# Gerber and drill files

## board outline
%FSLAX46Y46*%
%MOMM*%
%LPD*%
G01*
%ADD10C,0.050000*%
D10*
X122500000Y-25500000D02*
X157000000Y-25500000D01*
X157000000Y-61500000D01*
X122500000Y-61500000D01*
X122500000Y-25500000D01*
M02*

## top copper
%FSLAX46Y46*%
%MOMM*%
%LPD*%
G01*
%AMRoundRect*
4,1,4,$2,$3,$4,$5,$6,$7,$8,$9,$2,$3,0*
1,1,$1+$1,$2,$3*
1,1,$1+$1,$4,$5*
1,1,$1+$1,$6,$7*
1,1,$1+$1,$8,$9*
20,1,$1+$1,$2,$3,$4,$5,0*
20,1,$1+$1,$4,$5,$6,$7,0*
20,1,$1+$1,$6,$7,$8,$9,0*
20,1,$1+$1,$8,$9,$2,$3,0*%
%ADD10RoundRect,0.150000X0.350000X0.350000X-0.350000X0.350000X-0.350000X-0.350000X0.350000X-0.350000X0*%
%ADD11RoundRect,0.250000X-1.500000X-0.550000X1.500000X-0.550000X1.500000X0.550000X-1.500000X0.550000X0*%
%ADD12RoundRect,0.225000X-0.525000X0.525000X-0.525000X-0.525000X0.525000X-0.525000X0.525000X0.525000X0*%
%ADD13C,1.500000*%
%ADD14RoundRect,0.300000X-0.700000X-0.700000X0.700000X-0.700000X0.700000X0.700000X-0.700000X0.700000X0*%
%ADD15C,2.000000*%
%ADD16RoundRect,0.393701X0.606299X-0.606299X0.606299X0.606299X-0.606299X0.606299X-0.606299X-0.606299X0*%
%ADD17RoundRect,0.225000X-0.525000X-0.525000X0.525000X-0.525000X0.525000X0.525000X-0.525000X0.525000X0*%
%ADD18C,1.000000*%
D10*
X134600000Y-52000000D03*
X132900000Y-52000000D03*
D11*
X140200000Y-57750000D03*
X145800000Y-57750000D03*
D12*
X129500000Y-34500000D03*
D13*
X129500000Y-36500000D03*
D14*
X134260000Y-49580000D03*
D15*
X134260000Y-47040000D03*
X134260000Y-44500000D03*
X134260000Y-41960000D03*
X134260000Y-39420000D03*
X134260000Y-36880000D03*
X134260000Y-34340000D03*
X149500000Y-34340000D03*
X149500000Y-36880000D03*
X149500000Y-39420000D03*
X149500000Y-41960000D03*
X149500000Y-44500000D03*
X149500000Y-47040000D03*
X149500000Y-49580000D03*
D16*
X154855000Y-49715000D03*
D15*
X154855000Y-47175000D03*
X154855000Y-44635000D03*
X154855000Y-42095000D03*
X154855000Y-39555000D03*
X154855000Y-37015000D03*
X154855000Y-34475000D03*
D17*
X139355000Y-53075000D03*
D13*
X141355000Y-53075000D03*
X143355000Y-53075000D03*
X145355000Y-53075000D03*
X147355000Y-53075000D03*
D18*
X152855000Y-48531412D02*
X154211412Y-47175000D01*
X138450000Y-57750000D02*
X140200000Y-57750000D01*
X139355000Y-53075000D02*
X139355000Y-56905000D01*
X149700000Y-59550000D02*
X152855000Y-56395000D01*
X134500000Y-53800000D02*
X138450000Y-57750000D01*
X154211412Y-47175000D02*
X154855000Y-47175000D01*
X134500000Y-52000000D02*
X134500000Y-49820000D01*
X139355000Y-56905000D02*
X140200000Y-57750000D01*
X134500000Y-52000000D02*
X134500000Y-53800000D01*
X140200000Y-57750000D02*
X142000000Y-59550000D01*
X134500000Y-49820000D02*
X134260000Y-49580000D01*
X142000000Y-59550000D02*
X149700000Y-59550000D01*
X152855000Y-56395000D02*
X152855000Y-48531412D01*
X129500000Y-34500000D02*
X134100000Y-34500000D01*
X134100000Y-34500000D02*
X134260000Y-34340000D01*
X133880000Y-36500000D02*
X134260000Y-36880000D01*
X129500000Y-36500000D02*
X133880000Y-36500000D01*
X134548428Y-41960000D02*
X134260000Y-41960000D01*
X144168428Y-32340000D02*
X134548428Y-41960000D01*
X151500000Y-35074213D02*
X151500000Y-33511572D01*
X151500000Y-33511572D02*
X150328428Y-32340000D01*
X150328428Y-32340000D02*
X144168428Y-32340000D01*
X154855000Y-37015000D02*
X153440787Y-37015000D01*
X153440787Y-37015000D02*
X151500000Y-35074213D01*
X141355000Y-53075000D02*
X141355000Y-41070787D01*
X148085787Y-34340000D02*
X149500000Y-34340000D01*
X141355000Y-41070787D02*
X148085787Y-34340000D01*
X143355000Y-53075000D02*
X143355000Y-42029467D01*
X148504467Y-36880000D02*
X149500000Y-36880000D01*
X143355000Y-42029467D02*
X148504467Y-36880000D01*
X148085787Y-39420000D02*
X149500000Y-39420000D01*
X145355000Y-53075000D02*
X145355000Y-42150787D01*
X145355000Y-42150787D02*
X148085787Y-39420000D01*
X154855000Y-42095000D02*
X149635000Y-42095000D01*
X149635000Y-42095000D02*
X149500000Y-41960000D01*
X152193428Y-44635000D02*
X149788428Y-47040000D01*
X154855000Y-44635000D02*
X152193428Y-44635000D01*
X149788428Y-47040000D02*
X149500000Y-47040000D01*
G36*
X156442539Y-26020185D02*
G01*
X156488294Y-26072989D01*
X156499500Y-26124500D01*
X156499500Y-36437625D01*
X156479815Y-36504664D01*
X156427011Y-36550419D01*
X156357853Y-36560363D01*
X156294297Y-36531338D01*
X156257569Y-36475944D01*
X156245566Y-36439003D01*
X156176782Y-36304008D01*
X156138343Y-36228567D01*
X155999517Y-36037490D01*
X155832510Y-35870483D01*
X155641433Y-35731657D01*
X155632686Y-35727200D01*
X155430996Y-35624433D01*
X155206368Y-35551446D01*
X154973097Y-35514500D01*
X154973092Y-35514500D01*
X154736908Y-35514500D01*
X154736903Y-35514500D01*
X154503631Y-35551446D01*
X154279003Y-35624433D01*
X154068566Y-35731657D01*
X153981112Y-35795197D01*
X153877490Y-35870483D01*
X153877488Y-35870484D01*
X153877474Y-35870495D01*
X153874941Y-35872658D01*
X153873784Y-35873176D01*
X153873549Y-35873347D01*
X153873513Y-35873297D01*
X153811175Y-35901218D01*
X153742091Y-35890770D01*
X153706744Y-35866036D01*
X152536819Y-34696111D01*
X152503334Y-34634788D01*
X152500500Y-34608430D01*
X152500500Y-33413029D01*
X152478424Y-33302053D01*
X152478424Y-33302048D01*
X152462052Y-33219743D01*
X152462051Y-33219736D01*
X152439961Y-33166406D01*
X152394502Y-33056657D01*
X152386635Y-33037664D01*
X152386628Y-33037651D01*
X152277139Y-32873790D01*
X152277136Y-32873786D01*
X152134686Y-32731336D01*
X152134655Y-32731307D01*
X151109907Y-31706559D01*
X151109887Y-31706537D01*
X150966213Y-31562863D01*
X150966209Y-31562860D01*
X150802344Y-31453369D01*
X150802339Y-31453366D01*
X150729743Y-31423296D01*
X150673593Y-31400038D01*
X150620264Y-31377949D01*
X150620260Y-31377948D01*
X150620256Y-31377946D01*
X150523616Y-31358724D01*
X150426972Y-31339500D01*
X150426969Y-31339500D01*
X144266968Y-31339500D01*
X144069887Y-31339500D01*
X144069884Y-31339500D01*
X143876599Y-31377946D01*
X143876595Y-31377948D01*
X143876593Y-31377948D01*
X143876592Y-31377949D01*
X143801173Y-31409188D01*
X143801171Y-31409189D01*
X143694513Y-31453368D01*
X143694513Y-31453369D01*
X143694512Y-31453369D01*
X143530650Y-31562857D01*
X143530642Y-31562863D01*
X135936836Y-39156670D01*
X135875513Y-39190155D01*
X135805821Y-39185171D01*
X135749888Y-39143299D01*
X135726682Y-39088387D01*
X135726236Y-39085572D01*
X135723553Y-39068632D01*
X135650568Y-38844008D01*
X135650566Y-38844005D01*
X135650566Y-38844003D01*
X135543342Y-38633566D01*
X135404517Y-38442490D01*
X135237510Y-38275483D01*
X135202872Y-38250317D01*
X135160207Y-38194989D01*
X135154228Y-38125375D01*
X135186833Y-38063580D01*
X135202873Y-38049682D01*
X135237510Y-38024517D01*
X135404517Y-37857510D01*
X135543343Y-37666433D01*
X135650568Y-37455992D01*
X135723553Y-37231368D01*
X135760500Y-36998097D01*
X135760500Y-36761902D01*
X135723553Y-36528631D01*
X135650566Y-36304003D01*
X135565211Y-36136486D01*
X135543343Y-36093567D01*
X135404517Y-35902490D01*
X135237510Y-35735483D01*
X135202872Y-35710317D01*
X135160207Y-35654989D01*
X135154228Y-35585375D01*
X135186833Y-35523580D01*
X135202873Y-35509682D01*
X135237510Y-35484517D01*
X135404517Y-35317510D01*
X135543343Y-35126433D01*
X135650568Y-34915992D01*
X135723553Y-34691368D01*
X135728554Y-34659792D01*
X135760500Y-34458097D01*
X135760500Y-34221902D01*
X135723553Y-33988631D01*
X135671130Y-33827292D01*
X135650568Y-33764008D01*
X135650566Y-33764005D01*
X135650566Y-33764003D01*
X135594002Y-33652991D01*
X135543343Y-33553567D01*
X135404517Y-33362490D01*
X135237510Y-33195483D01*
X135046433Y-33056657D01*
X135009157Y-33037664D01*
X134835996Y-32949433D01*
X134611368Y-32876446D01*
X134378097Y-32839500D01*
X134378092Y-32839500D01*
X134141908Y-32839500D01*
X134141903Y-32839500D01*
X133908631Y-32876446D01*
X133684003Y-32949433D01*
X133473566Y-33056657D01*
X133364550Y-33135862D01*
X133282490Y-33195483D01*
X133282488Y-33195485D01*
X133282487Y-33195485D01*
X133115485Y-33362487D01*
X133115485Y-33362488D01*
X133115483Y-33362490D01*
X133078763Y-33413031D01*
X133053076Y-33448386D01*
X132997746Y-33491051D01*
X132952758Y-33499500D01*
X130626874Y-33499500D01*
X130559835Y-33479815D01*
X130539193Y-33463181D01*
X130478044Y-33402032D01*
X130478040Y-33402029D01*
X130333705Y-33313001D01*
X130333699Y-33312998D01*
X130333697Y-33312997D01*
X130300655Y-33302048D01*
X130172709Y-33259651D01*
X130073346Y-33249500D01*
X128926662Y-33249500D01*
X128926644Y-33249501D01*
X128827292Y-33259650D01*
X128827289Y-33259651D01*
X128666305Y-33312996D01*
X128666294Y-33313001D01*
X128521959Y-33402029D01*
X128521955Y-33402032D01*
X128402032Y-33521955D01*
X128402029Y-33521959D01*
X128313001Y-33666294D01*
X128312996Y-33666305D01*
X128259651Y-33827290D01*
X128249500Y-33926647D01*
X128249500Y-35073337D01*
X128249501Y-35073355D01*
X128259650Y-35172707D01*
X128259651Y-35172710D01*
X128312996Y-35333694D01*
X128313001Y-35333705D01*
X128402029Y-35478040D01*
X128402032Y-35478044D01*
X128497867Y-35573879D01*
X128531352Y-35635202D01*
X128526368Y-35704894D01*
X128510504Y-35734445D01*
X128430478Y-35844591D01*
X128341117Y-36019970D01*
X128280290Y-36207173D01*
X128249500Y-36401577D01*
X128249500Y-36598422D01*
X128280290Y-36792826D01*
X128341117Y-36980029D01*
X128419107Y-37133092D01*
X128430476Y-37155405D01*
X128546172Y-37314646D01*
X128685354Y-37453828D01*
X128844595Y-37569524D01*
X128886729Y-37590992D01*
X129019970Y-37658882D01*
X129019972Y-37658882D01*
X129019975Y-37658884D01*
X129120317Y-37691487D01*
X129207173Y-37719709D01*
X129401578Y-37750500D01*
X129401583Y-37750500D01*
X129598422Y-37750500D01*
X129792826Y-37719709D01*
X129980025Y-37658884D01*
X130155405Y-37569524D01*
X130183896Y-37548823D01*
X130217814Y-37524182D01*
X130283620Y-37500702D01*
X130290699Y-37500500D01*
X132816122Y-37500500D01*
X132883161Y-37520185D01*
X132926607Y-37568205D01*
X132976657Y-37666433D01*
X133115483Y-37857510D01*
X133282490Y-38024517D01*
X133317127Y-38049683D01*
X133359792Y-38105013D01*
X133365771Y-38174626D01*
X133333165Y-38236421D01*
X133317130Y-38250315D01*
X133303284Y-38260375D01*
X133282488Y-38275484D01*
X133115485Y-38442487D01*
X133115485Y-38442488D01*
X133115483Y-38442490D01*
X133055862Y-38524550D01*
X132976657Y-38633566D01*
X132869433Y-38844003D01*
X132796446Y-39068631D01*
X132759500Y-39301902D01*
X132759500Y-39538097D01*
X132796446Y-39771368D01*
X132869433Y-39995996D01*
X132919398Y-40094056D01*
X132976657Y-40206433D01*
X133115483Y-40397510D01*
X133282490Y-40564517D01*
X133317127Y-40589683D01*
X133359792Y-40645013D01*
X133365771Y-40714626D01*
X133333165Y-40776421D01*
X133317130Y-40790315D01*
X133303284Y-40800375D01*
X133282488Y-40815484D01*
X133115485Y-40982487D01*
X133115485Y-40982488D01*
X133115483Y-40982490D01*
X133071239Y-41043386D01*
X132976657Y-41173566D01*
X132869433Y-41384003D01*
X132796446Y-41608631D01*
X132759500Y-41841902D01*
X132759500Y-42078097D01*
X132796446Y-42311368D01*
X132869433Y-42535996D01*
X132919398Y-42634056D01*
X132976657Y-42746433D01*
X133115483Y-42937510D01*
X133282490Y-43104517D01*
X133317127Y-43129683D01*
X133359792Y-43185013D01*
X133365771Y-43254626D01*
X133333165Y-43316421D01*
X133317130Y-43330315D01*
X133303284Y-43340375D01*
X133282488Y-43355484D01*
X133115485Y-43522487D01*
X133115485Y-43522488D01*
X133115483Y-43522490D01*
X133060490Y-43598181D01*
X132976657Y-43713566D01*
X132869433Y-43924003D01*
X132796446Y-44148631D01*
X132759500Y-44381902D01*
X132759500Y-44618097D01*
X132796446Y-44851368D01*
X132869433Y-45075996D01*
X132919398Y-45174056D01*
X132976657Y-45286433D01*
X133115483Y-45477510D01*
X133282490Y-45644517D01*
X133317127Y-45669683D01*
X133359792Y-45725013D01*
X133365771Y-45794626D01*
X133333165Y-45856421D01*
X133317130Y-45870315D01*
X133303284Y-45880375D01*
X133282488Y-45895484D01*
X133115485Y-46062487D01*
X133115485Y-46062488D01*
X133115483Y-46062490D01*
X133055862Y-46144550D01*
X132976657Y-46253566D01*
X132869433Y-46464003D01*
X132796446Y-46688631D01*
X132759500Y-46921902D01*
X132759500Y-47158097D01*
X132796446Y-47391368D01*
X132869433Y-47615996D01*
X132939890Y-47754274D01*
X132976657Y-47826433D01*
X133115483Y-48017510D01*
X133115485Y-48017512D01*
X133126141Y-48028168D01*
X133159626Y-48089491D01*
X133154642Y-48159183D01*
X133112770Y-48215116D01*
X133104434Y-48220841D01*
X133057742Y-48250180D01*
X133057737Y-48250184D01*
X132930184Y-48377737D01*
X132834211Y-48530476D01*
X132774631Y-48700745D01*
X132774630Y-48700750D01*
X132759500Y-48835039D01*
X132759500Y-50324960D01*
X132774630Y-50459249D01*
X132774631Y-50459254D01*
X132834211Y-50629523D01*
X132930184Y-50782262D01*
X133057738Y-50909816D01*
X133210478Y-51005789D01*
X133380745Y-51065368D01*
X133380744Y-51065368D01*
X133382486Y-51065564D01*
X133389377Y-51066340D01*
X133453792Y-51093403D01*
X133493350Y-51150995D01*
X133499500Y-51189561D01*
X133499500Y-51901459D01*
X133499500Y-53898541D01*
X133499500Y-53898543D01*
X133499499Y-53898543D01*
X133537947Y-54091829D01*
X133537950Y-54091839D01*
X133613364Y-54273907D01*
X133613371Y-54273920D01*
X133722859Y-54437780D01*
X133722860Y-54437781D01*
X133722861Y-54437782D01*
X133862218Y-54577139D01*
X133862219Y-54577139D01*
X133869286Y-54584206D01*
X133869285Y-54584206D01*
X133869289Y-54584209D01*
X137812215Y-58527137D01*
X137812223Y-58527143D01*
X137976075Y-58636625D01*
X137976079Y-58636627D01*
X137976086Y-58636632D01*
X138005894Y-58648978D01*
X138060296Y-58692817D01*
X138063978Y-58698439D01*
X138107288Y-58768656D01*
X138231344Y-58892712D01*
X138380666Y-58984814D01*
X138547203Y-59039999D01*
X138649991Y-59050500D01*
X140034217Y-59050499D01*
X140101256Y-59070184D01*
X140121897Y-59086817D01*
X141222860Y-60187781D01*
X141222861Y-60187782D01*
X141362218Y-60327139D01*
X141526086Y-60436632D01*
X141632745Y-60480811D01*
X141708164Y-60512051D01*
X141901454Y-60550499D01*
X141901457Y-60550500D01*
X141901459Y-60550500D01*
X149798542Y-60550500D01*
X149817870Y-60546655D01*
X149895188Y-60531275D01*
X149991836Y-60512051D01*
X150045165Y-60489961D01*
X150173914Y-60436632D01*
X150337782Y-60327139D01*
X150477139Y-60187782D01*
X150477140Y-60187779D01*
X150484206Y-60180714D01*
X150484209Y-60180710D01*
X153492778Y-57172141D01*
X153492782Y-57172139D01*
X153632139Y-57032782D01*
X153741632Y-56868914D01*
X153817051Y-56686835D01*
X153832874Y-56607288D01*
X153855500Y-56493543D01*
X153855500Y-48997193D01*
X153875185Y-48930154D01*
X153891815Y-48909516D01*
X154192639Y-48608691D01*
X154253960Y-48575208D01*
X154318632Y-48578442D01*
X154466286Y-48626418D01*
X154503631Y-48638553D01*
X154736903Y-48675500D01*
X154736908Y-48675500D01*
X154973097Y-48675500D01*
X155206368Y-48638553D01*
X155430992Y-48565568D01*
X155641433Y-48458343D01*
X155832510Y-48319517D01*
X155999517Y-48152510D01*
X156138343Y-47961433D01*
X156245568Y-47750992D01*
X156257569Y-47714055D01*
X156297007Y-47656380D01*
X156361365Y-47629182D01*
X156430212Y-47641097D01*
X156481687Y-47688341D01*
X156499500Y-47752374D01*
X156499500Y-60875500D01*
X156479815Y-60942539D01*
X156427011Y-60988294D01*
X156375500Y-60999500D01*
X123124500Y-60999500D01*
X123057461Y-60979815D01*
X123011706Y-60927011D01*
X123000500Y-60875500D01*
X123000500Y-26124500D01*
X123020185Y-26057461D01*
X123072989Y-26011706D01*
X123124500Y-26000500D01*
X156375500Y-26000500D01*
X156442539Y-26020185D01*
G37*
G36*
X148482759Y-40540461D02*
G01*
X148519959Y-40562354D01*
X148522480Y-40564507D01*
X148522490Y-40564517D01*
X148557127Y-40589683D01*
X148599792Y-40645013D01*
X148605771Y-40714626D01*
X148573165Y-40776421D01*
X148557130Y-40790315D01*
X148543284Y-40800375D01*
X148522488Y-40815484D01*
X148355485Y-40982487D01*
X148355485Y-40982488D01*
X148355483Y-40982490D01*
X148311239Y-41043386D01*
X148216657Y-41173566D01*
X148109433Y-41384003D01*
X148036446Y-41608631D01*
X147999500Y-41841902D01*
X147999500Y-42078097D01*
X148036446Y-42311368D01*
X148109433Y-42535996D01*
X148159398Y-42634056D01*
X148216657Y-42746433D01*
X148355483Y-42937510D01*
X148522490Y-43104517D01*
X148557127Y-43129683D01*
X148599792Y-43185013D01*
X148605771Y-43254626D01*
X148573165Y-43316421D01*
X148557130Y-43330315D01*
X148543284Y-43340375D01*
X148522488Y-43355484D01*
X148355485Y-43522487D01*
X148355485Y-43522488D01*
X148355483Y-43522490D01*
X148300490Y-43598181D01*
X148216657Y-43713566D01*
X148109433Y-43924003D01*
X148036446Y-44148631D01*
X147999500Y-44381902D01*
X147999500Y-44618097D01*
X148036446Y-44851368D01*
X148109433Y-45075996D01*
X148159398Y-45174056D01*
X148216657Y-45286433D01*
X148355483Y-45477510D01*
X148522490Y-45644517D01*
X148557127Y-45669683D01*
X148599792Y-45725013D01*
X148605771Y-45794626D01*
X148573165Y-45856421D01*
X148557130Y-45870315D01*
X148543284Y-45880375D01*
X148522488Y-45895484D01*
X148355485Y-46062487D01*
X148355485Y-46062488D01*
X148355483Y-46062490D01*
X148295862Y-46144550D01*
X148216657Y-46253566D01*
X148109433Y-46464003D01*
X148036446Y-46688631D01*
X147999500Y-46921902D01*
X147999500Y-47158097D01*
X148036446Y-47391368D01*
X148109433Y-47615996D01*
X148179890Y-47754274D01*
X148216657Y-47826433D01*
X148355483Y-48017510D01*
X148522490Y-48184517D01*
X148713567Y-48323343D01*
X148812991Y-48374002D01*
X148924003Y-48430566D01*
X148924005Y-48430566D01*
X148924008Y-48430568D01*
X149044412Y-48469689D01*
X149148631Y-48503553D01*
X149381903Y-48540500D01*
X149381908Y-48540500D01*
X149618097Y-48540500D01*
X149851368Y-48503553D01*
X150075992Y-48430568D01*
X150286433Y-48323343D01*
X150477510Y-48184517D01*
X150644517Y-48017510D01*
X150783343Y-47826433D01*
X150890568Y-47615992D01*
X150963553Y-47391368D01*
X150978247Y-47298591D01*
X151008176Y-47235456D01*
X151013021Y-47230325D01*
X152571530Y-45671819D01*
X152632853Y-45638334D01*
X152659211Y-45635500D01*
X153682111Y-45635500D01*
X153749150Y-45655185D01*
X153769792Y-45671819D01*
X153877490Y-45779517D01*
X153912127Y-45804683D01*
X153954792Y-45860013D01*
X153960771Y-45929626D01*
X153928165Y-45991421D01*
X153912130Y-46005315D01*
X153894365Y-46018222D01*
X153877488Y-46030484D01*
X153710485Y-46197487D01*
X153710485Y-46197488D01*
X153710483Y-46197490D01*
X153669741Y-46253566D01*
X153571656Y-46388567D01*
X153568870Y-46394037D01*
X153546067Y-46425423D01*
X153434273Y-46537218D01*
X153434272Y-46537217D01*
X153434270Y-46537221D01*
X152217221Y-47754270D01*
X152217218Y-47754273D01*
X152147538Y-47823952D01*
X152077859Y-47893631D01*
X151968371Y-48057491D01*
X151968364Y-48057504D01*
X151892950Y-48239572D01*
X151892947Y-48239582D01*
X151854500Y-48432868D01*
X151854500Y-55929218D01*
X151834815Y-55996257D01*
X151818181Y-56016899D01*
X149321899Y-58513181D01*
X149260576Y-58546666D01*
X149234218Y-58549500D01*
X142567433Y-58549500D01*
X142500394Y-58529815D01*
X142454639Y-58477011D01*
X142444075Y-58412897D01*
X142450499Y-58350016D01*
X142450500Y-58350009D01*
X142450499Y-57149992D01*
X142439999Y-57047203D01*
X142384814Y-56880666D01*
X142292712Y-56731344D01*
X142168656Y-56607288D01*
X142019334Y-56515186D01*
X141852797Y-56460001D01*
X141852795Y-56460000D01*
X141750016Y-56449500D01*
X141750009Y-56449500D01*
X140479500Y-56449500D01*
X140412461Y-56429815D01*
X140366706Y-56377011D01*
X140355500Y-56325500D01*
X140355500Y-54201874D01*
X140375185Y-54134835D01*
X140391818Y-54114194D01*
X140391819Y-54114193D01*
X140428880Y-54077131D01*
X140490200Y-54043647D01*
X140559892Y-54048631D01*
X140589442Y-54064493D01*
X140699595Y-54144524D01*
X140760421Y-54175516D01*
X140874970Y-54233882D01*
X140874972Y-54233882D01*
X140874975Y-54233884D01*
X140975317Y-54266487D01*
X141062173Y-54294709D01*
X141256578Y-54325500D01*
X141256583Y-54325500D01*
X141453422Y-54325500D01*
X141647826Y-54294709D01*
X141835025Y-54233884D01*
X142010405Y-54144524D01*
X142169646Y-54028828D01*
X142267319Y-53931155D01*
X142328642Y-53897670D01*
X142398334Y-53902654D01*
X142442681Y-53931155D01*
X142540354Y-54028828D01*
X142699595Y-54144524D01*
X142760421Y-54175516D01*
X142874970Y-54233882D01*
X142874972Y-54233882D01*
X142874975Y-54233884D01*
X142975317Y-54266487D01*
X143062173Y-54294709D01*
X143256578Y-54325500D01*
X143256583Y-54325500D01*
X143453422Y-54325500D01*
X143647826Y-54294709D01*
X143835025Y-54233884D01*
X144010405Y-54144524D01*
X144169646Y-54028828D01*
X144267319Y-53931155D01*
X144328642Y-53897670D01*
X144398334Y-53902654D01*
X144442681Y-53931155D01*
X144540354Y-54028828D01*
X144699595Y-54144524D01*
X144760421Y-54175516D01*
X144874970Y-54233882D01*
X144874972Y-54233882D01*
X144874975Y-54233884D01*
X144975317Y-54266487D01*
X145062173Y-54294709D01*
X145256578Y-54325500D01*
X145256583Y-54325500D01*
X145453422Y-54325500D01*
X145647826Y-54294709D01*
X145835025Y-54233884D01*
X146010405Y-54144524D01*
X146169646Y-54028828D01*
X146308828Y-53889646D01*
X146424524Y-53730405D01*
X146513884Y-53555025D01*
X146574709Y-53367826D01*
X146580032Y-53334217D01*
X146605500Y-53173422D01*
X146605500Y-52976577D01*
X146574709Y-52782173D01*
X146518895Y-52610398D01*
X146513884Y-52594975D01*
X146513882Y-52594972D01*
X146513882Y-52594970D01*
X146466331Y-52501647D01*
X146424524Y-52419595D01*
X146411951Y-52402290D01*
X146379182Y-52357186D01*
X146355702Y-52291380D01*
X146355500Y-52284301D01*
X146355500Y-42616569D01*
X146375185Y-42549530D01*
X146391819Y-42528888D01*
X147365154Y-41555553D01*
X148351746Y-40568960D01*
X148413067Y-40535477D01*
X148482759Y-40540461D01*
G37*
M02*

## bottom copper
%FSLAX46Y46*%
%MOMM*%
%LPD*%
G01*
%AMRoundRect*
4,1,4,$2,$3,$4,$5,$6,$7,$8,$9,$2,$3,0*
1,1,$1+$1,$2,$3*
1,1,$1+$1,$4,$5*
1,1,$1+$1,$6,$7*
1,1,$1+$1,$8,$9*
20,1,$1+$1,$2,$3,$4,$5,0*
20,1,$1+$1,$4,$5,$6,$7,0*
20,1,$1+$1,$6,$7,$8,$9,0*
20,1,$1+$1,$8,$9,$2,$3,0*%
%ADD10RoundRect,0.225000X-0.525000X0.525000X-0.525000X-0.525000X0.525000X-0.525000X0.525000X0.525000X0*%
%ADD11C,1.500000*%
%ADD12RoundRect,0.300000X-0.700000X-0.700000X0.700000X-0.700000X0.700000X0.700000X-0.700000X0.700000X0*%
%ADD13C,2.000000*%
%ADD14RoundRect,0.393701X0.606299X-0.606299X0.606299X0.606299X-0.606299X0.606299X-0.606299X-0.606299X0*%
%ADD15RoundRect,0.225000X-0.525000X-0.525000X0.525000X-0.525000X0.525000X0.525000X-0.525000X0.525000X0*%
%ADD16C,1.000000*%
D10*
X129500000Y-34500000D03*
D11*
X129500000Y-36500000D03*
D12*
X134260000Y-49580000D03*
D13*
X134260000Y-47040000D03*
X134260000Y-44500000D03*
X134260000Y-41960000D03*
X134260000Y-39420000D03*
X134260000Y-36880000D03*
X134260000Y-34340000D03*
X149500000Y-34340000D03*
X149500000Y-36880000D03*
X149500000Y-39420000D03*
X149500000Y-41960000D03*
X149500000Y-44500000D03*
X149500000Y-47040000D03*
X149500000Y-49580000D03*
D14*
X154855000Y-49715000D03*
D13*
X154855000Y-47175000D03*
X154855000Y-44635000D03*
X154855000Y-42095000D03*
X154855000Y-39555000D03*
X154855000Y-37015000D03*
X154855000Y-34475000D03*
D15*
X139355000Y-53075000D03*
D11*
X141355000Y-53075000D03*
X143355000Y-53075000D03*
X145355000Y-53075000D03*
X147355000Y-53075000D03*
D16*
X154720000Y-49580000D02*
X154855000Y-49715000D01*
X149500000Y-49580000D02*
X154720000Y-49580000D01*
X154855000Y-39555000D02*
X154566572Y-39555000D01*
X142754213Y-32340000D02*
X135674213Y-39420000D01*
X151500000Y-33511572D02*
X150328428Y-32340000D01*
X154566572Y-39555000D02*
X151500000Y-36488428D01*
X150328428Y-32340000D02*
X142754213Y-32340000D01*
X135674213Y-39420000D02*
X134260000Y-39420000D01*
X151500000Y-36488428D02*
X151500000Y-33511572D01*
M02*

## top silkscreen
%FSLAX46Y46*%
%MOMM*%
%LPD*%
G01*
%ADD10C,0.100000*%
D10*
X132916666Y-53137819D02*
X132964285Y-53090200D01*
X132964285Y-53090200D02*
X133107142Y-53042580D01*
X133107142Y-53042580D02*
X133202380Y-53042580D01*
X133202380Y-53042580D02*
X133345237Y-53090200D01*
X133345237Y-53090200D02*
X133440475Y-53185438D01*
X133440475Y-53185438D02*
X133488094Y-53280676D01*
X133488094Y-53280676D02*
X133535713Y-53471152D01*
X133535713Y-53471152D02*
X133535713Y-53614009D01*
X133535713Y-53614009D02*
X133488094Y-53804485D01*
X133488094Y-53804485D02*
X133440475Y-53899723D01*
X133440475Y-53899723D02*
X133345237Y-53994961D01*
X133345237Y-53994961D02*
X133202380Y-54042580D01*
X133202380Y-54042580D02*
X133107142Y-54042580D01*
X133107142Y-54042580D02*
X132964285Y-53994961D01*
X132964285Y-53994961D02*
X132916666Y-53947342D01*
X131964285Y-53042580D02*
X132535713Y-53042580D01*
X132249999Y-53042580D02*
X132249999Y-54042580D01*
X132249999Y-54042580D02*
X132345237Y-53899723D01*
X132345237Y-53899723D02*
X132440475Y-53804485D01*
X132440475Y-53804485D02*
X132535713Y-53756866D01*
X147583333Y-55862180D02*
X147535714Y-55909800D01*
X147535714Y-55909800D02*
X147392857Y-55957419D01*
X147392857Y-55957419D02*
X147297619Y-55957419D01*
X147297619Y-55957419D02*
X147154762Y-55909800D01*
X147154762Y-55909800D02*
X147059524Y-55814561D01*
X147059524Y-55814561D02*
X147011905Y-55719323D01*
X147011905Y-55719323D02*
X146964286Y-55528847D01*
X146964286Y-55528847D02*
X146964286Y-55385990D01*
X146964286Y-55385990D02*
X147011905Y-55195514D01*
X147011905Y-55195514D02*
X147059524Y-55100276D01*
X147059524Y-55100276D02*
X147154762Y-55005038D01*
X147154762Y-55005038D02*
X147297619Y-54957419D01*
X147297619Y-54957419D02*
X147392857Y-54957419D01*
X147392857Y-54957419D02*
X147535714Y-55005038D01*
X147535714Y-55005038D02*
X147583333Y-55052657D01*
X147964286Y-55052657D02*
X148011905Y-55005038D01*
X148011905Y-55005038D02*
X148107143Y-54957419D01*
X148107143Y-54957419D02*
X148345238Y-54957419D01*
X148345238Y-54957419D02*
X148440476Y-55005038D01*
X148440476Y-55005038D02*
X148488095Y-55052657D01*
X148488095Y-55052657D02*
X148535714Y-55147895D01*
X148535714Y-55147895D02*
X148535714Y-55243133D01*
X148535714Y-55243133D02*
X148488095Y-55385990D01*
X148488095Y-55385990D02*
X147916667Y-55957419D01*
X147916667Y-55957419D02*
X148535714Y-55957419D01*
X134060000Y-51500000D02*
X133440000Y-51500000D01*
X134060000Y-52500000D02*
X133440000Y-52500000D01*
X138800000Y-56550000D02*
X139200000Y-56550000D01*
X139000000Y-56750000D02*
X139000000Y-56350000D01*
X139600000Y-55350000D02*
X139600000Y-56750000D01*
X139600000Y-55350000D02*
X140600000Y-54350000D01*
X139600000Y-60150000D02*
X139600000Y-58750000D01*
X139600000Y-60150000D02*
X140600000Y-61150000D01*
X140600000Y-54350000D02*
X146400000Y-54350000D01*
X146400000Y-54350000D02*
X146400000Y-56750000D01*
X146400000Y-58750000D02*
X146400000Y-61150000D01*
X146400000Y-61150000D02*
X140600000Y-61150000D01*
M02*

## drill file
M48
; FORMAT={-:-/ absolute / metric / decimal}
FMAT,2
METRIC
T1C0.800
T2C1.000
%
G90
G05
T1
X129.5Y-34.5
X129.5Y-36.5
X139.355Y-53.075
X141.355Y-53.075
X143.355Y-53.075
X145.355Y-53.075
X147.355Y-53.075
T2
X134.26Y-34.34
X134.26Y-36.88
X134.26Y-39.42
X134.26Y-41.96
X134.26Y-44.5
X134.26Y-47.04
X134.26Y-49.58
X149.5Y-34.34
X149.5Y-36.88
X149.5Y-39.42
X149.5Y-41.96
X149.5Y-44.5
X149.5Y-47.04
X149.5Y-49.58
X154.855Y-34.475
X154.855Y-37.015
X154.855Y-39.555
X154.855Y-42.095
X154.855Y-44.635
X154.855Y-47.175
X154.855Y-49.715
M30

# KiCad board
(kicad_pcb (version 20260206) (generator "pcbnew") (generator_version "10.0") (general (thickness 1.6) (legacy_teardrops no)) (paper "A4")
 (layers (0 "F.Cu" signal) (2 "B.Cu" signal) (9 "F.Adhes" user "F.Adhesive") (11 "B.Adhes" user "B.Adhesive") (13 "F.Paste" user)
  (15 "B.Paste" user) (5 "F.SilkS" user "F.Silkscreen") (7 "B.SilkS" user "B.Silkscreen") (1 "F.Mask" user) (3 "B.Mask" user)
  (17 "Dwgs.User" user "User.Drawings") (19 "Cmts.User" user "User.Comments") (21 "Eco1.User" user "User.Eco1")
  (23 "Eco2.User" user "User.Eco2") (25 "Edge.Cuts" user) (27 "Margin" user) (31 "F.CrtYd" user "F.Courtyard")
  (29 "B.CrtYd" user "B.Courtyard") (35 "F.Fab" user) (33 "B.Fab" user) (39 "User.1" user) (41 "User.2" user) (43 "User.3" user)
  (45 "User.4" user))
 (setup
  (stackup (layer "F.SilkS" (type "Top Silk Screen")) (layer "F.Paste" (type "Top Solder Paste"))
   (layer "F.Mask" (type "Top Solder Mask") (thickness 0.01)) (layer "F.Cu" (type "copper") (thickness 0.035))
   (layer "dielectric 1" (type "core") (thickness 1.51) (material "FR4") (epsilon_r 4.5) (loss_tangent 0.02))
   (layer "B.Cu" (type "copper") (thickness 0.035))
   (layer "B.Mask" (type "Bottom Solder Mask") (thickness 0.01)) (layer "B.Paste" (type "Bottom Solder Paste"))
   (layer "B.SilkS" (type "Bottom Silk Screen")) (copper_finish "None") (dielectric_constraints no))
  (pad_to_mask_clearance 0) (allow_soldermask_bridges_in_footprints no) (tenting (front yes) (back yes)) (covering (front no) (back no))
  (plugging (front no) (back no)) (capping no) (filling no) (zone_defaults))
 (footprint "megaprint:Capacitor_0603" (layer "F.Cu") (at 133.75 52 180)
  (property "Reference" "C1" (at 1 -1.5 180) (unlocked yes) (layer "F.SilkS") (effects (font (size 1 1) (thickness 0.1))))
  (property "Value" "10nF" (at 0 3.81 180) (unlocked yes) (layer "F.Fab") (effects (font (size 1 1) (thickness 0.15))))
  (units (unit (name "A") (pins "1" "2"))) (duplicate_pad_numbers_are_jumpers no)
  (fp_line (start -0.31 0.5) (end 0.31 0.5) (stroke (width 0.1) (type default)) (layer "F.SilkS"))
  (fp_line (start -0.31 -0.5) (end 0.31 -0.5) (stroke (width 0.1) (type default)) (layer "F.SilkS"))
  (pad "1" smd roundrect (at -0.85 0 180) (size 1 1) (layers "F.Cu" "F.Mask" "F.Paste") (roundrect_rratio 0.15) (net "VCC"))
  (pad "2" smd roundrect (at 0.85 0 180) (size 1 1) (layers "F.Cu" "F.Mask" "F.Paste") (roundrect_rratio 0.15) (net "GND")))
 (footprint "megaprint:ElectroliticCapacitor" (layer "F.Cu") (at 143 57.75)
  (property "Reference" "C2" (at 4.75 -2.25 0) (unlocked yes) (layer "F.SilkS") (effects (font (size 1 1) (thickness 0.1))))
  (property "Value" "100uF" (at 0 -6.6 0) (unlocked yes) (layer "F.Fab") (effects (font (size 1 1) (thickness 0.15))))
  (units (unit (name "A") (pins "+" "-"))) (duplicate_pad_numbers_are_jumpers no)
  (fp_line (start -4.2 -1.2) (end -3.8 -1.2) (stroke (width 0.1) (type default)) (layer "F.SilkS"))
  (fp_line (start -4 -1) (end -4 -1.4) (stroke (width 0.1) (type default)) (layer "F.SilkS"))
  (fp_line (start -3.4 -2.4) (end -3.4 -1) (stroke (width 0.1) (type default)) (layer "F.SilkS"))
  (fp_line (start -3.4 -2.4) (end -2.4 -3.4) (stroke (width 0.1) (type default)) (layer "F.SilkS"))
  (fp_line (start -3.4 2.4) (end -3.4 1) (stroke (width 0.1) (type default)) (layer "F.SilkS"))
  (fp_line (start -3.4 2.4) (end -2.4 3.4) (stroke (width 0.1) (type default)) (layer "F.SilkS"))
  (fp_line (start -2.4 -3.4) (end 3.4 -3.4) (stroke (width 0.1) (type default)) (layer "F.SilkS"))
  (fp_line (start 3.4 -3.4) (end 3.4 -1) (stroke (width 0.1) (type default)) (layer "F.SilkS"))
  (fp_line (start 3.4 1) (end 3.4 3.4) (stroke (width 0.1) (type default)) (layer "F.SilkS"))
  (fp_line (start 3.4 3.4) (end -2.4 3.4) (stroke (width 0.1) (type default)) (layer "F.SilkS"))
  (pad "+" smd roundrect (at -2.8 0) (size 3.5 1.6) (layers "F.Cu" "F.Mask" "F.Paste") (roundrect_rratio 0.15625) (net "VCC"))
  (pad "-" smd roundrect (at 2.8 0) (size 3.5 1.6) (layers "F.Cu" "F.Mask" "F.Paste") (roundrect_rratio 0.15625) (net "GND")))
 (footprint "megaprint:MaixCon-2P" (layer "B.Cu") (at 129.5 35.5 -90)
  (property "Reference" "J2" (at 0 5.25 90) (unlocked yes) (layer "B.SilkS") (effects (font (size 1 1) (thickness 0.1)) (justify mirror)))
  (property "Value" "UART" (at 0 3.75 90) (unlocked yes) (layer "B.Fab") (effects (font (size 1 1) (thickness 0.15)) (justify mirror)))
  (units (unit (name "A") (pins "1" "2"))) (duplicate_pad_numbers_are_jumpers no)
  (pad "1" thru_hole roundrect (at -1 0 270) (size 1.5 1.5) (drill 0.8) (layers "*.Cu" "*.Mask") (remove_unused_layers no)
   (roundrect_rratio 0.15) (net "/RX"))
  (pad "2" thru_hole circle (at 1 0 270) (size 1.5 1.5) (drill 0.8) (layers "*.Cu" "*.Mask") (remove_unused_layers no) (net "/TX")
   (thermal_bridge_angle 90)))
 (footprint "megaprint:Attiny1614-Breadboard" (layer "B.Cu") (at 141.88 41.96)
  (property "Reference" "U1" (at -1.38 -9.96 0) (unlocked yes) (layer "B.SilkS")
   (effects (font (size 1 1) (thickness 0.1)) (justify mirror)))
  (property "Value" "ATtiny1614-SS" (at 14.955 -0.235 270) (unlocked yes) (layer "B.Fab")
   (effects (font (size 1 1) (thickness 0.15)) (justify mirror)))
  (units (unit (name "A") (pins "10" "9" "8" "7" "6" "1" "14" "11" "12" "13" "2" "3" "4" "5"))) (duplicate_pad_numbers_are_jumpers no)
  (pad "1" thru_hole roundrect (at -7.62 7.62) (size 2 2) (drill 1) (layers "*.Cu" "*.Mask") (remove_unused_layers no)
   (roundrect_rratio 0.15) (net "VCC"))
  (pad "2" thru_hole circle (at -7.62 5.08) (size 2 2) (drill 1) (layers "*.Cu" "*.Mask") (remove_unused_layers no)
   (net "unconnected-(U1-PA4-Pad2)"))
  (pad "3" thru_hole circle (at -7.62 2.54) (size 2 2) (drill 1) (layers "*.Cu" "*.Mask") (remove_unused_layers no)
   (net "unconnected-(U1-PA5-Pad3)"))
  (pad "4" thru_hole circle (at -7.62 0) (size 2 2) (drill 1) (layers "*.Cu" "*.Mask") (remove_unused_layers no) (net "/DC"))
  (pad "5" thru_hole circle (at -7.62 -2.54) (size 2 2) (drill 1) (layers "*.Cu" "*.Mask") (remove_unused_layers no) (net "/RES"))
  (pad "6" thru_hole circle (at -7.62 -5.08) (size 2 2) (drill 1) (layers "*.Cu" "*.Mask") (remove_unused_layers no) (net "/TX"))
  (pad "7" thru_hole circle (at -7.62 -7.62) (size 2 2) (drill 1) (layers "*.Cu" "*.Mask") (remove_unused_layers no) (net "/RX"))
  (pad "8" thru_hole circle (at 7.62 -7.62) (size 2 2) (drill 1) (layers "*.Cu" "*.Mask") (remove_unused_layers no) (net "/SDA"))
  (pad "9" thru_hole circle (at 7.62 -5.08) (size 2 2) (drill 1) (layers "*.Cu" "*.Mask") (remove_unused_layers no) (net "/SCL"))
  (pad "10" thru_hole circle (at 7.62 -2.54) (size 2 2) (drill 1) (layers "*.Cu" "*.Mask") (remove_unused_layers no) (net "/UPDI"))
  (pad "11" thru_hole circle (at 7.62 0) (size 2 2) (drill 1) (layers "*.Cu" "*.Mask") (remove_unused_layers no) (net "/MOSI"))
  (pad "12" thru_hole circle (at 7.62 2.54) (size 2 2) (drill 1) (layers "*.Cu" "*.Mask") (remove_unused_layers no)
   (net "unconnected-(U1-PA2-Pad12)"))
  (pad "13" thru_hole circle (at 7.62 5.08) (size 2 2) (drill 1) (layers "*.Cu" "*.Mask") (remove_unused_layers no) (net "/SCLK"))
  (pad "14" thru_hole circle (at 7.62 7.62) (size 2 2) (drill 1) (layers "*.Cu" "*.Mask") (remove_unused_layers no) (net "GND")))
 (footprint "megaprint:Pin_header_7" (layer "B.Cu") (at 154.855 42.145 90)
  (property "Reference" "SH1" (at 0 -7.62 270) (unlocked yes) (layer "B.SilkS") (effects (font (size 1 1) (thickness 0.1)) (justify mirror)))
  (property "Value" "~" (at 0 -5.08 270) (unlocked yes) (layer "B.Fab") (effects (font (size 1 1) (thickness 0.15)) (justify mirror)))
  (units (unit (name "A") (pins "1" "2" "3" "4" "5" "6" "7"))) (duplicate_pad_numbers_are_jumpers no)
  (pad "1" thru_hole roundrect (at -7.57 0 90) (size 2 2) (drill 1) (layers "*.Cu" "*.Mask") (remove_unused_layers no)
   (roundrect_rratio 0.1968503937) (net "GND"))
  (pad "2" thru_hole circle (at -5.03 0 90) (size 2 2) (drill 1) (layers "*.Cu" "*.Mask") (remove_unused_layers no) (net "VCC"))
  (pad "3" thru_hole circle (at -2.49 0 90) (size 2 2) (drill 1) (layers "*.Cu" "*.Mask") (remove_unused_layers no) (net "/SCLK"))
  (pad "4" thru_hole circle (at 0.05 0 90) (size 2 2) (drill 1) (layers "*.Cu" "*.Mask") (remove_unused_layers no) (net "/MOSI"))
  (pad "5" thru_hole circle (at 2.59 0 90) (size 2 2) (drill 1) (layers "*.Cu" "*.Mask") (remove_unused_layers no) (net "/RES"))
  (pad "6" thru_hole circle (at 5.13 0 90) (size 2 2) (drill 1) (layers "*.Cu" "*.Mask") (remove_unused_layers no) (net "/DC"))
  (pad "7" thru_hole circle (at 7.67 0 90) (size 2 2) (drill 1) (layers "*.Cu" "*.Mask") (remove_unused_layers no) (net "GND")))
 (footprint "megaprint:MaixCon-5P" (layer "B.Cu") (at 143.355 53.075)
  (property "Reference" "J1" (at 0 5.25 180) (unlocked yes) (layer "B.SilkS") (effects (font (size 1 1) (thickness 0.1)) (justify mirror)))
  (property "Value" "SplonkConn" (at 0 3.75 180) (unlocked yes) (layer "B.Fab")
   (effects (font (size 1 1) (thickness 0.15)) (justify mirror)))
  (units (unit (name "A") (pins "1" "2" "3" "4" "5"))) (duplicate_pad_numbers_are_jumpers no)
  (pad "1" thru_hole roundrect (at -4 0) (size 1.5 1.5) (drill 0.8) (layers "*.Cu" "*.Mask") (remove_unused_layers no)
   (roundrect_rratio 0.15) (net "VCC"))
  (pad "2" thru_hole circle (at -2 0) (size 1.5 1.5) (drill 0.8) (layers "*.Cu" "*.Mask") (remove_unused_layers no) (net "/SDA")
   (thermal_bridge_angle 90))
  (pad "3" thru_hole circle (at 0 0) (size 1.5 1.5) (drill 0.8) (layers "*.Cu" "*.Mask") (remove_unused_layers no) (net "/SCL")
   (thermal_bridge_angle 90))
  (pad "4" thru_hole circle (at 2 0) (size 1.5 1.5) (drill 0.8) (layers "*.Cu" "*.Mask") (remove_unused_layers no) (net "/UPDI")
   (thermal_bridge_angle 90))
  (pad "5" thru_hole circle (at 4 0) (size 1.5 1.5) (drill 0.8) (layers "*.Cu" "*.Mask") (remove_unused_layers no) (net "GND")
   (thermal_bridge_angle 90)))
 (gr_rect (start 122.5 25.5) (end 157 61.5) (stroke (width 0.05) (type solid)) (fill no) (layer "Edge.Cuts"))
 (segment (start 152.855 48.531412) (end 154.211412 47.175) (width 1) (layer "F.Cu") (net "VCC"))
 (segment (start 138.45 57.75) (end 140.2 57.75) (width 1) (layer "F.Cu") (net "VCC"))
 (segment (start 139.355 53.075) (end 139.355 56.905) (width 1) (layer "F.Cu") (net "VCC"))
 (segment (start 149.7 59.55) (end 152.855 56.395) (width 1) (layer "F.Cu") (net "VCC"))
 (segment (start 134.5 53.8) (end 138.45 57.75) (width 1) (layer "F.Cu") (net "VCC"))
 (segment (start 154.211412 47.175) (end 154.855 47.175) (width 1) (layer "F.Cu") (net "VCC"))
 (segment (start 134.5 52) (end 134.5 49.82) (width 1) (layer "F.Cu") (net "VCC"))
 (segment (start 139.355 56.905) (end 140.2 57.75) (width 1) (layer "F.Cu") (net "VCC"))
 (segment (start 134.5 52) (end 134.5 53.8) (width 1) (layer "F.Cu") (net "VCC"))
 (segment (start 140.2 57.75) (end 142 59.55) (width 1) (layer "F.Cu") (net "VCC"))
 (segment (start 134.5 49.82) (end 134.26 49.58) (width 1) (layer "F.Cu") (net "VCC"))
 (segment (start 142 59.55) (end 149.7 59.55) (width 1) (layer "F.Cu") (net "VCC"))
 (segment (start 152.855 56.395) (end 152.855 48.531412) (width 1) (layer "F.Cu") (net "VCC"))
 (segment (start 154.72 49.58) (end 154.855 49.715) (width 1) (layer "B.Cu") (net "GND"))
 (segment (start 149.5 49.58) (end 154.72 49.58) (width 1) (layer "B.Cu") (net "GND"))
 (segment (start 129.5 34.5) (end 134.1 34.5) (width 1) (layer "F.Cu") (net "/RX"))
 (segment (start 134.1 34.5) (end 134.26 34.34) (width 1) (layer "F.Cu") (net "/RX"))
 (segment (start 133.88 36.5) (end 134.26 36.88) (width 1) (layer "F.Cu") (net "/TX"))
 (segment (start 129.5 36.5) (end 133.88 36.5) (width 1) (layer "F.Cu") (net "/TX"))
 (segment (start 134.548428 41.96) (end 134.26 41.96) (width 1) (layer "F.Cu") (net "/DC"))
 (segment (start 144.168428 32.34) (end 134.548428 41.96) (width 1) (layer "F.Cu") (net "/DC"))
 (segment (start 151.5 35.074213) (end 151.5 33.511572) (width 1) (layer "F.Cu") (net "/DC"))
 (segment (start 151.5 33.511572) (end 150.328428 32.34) (width 1) (layer "F.Cu") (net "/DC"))
 (segment (start 150.328428 32.34) (end 144.168428 32.34) (width 1) (layer "F.Cu") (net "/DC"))
 (segment (start 154.855 37.015) (end 153.440787 37.015) (width 1) (layer "F.Cu") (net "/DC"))
 (segment (start 153.440787 37.015) (end 151.5 35.074213) (width 1) (layer "F.Cu") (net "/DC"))
 (segment (start 154.855 39.555) (end 154.566572 39.555) (width 1) (layer "B.Cu") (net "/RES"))
 (segment (start 142.754213 32.34) (end 135.674213 39.42) (width 1) (layer "B.Cu") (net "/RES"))
 (segment (start 151.5 33.511572) (end 150.328428 32.34) (width 1) (layer "B.Cu") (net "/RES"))
 (segment (start 154.566572 39.555) (end 151.5 36.488428) (width 1) (layer "B.Cu") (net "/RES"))
 (segment (start 150.328428 32.34) (end 142.754213 32.34) (width 1) (layer "B.Cu") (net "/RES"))
 (segment (start 135.674213 39.42) (end 134.26 39.42) (width 1) (layer "B.Cu") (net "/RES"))
 (segment (start 151.5 36.488428) (end 151.5 33.511572) (width 1) (layer "B.Cu") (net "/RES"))
 (segment (start 141.355 53.075) (end 141.355 41.070787) (width 1) (layer "F.Cu") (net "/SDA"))
 (segment (start 148.085787 34.34) (end 149.5 34.34) (width 1) (layer "F.Cu") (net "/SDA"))
 (segment (start 141.355 41.070787) (end 148.085787 34.34) (width 1) (layer "F.Cu") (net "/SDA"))
 (segment (start 143.355 53.075) (end 143.355 42.029467) (width 1) (layer "F.Cu") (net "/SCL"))
 (segment (start 148.504467 36.88) (end 149.5 36.88) (width 1) (layer "F.Cu") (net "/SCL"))
 (segment (start 143.355 42.029467) (end 148.504467 36.88) (width 1) (layer "F.Cu") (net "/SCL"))
 (segment (start 148.085787 39.42) (end 149.5 39.42) (width 1) (layer "F.Cu") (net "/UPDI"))
 (segment (start 145.355 53.075) (end 145.355 42.150787) (width 1) (layer "F.Cu") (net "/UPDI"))
 (segment (start 145.355 42.150787) (end 148.085787 39.42) (width 1) (layer "F.Cu") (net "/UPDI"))
 (segment (start 154.855 42.095) (end 149.635 42.095) (width 1) (layer "F.Cu") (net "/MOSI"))
 (segment (start 149.635 42.095) (end 149.5 41.96) (width 1) (layer "F.Cu") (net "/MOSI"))
 (segment (start 152.193428 44.635) (end 149.788428 47.04) (width 1) (layer "F.Cu") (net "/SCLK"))
 (segment (start 154.855 44.635) (end 152.193428 44.635) (width 1) (layer "F.Cu") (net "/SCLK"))
 (segment (start 149.788428 47.04) (end 149.5 47.04) (width 1) (layer "F.Cu") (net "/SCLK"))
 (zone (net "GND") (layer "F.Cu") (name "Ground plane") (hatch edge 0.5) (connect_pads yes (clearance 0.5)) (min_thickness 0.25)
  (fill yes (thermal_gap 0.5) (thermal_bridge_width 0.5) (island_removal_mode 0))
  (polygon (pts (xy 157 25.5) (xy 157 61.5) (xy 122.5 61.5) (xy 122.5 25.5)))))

